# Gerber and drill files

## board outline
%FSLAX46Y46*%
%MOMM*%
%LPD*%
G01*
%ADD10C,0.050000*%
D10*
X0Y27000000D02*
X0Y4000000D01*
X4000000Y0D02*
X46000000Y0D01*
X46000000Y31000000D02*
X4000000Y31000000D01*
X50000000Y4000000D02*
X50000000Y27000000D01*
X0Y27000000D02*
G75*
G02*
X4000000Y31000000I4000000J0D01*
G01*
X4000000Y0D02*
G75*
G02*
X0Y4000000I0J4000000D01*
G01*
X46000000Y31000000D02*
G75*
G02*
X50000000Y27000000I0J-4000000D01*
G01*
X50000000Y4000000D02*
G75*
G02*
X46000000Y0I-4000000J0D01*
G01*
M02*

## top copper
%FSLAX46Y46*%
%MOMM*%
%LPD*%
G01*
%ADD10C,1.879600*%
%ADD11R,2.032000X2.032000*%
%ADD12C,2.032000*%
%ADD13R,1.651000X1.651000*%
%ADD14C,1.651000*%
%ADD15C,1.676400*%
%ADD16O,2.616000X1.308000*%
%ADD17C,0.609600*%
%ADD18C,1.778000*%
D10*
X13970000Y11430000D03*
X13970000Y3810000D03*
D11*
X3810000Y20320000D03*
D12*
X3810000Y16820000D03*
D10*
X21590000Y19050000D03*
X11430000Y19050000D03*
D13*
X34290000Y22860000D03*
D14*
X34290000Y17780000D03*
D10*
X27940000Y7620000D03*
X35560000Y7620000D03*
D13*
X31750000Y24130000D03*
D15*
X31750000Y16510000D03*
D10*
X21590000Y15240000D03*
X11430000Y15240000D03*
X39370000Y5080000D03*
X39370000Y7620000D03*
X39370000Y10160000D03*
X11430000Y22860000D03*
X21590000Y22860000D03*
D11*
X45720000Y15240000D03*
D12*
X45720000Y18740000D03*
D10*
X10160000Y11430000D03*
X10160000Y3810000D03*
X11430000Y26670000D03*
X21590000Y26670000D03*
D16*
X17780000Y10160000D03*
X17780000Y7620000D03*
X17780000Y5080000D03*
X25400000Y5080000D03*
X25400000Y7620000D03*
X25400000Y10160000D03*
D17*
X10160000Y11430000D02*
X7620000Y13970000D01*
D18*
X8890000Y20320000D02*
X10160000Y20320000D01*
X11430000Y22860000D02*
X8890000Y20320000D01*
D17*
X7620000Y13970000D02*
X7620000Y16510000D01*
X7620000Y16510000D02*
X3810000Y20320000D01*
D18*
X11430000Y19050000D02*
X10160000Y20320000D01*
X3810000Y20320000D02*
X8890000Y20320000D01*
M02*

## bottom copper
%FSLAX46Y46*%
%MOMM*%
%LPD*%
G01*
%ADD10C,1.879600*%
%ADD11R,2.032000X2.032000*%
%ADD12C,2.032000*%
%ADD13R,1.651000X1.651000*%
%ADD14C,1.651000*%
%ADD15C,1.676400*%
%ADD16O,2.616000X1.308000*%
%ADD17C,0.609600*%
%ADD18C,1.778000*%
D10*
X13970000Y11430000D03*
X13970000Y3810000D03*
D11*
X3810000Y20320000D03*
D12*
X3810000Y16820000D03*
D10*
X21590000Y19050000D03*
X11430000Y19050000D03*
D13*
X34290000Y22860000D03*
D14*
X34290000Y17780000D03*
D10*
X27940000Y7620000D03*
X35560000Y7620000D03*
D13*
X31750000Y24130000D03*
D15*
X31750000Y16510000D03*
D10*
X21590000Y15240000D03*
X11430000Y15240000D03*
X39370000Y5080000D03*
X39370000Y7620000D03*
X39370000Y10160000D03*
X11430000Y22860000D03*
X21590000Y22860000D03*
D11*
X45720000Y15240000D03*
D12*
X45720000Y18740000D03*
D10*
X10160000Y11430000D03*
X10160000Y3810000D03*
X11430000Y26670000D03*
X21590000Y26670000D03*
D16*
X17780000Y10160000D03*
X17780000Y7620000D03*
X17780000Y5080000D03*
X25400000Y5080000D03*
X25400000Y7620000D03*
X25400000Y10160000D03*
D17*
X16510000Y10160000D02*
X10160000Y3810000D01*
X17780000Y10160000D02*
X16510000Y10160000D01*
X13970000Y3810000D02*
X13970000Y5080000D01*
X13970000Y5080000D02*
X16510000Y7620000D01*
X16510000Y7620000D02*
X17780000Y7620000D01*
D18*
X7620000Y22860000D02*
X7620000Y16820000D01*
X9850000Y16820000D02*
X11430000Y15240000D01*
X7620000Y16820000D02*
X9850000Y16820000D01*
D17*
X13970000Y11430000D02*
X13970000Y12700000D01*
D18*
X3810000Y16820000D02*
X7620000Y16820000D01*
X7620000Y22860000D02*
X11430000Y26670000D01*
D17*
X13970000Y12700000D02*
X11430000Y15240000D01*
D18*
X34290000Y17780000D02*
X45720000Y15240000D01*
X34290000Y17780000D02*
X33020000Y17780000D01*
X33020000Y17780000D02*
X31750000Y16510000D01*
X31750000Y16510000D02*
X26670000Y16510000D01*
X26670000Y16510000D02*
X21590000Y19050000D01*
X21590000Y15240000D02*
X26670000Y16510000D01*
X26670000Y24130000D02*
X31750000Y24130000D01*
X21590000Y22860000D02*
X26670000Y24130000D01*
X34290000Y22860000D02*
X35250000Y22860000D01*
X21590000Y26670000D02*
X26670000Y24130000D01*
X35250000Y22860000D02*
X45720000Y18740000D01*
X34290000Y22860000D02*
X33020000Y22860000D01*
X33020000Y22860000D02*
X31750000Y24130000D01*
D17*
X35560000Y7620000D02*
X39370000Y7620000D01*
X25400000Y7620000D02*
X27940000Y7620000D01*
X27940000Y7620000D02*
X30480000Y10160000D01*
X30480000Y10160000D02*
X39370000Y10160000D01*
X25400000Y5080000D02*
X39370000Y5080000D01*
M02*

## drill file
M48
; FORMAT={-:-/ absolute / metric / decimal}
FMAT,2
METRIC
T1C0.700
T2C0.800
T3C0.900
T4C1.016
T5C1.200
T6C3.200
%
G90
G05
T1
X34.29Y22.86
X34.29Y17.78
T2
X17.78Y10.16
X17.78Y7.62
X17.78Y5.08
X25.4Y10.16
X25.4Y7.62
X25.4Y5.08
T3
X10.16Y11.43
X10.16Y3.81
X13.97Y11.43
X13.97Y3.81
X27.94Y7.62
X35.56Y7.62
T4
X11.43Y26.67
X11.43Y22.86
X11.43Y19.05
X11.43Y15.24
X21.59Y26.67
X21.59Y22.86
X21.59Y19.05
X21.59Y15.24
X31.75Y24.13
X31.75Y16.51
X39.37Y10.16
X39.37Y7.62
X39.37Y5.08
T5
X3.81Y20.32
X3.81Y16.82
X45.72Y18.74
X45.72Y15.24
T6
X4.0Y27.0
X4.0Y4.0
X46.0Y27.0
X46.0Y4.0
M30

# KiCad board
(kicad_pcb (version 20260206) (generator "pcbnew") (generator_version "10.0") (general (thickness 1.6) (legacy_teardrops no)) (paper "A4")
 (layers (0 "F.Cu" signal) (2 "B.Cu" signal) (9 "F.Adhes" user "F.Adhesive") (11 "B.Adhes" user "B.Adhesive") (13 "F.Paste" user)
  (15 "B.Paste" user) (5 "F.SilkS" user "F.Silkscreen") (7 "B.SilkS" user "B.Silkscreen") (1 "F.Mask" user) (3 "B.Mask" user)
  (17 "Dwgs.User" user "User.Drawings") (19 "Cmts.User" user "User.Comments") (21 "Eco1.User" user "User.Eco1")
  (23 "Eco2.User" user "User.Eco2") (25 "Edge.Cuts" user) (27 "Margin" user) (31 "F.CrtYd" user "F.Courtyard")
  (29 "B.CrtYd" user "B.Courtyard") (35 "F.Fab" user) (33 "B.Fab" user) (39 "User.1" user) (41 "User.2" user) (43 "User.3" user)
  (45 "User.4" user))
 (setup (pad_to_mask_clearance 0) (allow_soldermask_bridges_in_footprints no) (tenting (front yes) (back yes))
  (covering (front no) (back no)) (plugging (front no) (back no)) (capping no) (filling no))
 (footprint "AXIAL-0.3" (layer "F.Cu") (at 13.97 -7.62 -90)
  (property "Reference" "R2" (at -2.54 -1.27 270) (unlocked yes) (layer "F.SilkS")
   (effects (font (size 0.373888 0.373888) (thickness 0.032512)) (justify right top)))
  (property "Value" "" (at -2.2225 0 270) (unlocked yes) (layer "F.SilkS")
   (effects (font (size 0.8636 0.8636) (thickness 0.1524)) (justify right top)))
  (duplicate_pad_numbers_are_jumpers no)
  (pad "P$1" thru_hole circle (at -3.81 0 270) (size 1.8796 1.8796) (drill 0.9) (layers "*.Cu" "*.Mask") (remove_unused_layers no)
   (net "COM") (solder_mask_margin 0.1016) (thermal_bridge_angle 0))
  (pad "P$2" thru_hole circle (at 3.81 0 270) (size 1.8796 1.8796) (drill 0.9) (layers "*.Cu" "*.Mask") (remove_unused_layers no) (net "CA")
   (solder_mask_margin 0.1016) (thermal_bridge_angle 0)))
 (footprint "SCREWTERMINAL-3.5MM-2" (layer "F.Cu") (at 3.81 -20.32 -90)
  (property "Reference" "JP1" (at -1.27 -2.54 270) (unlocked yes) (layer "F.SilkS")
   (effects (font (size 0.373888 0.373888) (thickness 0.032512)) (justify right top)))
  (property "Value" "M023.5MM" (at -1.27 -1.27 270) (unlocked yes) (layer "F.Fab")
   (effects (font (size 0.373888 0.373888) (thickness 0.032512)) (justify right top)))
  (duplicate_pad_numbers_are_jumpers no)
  (pad "1" thru_hole rect (at 0 0 270) (size 2.032 2.032) (drill 1.2) (layers "*.Cu" "*.Mask") (remove_unused_layers no) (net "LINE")
   (solder_mask_margin 0.1016) (thermal_bridge_angle 0))
  (pad "2" thru_hole circle (at 3.5 0 270) (size 2.032 2.032) (drill 1.2) (layers "*.Cu" "*.Mask") (remove_unused_layers no) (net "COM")
   (solder_mask_margin 0.1016) (thermal_bridge_angle 0)))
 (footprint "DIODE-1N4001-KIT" (layer "F.Cu") (at 16.51 -19.05 180)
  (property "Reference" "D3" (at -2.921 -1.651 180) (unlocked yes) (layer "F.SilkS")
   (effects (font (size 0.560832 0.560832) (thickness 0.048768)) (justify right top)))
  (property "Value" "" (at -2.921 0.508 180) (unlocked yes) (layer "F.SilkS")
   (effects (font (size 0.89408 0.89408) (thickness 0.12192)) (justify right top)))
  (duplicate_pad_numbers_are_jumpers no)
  (pad "A" thru_hole circle (at -5.08 0 180) (size 1.8796 1.8796) (drill 1.016) (layers "*.Cu") (remove_unused_layers no) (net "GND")
   (solder_mask_margin 0.1016) (thermal_bridge_angle 0))
  (pad "C" thru_hole circle (at 5.08 0 180) (size 1.8796 1.8796) (drill 1.016) (layers "*.Cu") (remove_unused_layers no) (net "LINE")
   (solder_mask_margin 0.1016) (thermal_bridge_angle 0)))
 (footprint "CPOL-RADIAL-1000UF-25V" (layer "F.Cu") (at 34.29 -20.32 90)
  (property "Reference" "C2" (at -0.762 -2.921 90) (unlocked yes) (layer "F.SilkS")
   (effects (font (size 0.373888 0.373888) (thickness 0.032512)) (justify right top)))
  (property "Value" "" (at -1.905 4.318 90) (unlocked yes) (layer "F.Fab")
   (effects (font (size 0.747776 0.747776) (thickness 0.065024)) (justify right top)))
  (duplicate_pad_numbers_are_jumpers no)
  (pad "1" thru_hole rect (at 2.54 0 90) (size 1.651 1.651) (drill 0.7) (layers "*.Cu" "*.Mask") (remove_unused_layers no) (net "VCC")
   (solder_mask_margin 0.1016) (thermal_bridge_angle 0))
  (pad "2" thru_hole circle (at -2.54 0 90) (size 1.651 1.651) (drill 0.7) (layers "*.Cu" "*.Mask") (remove_unused_layers no) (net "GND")
   (solder_mask_margin 0.1016) (thermal_bridge_angle 0)))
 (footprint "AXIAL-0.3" (layer "F.Cu") (at 31.75 -7.62)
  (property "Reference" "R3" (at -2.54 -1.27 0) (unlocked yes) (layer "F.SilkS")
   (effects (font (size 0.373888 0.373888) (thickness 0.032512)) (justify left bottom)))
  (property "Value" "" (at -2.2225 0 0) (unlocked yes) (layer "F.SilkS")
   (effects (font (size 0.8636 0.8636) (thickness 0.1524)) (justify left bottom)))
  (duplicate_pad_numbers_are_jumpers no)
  (pad "P$1" thru_hole circle (at -3.81 0) (size 1.8796 1.8796) (drill 0.9) (layers "*.Cu" "*.Mask") (remove_unused_layers no) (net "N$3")
   (solder_mask_margin 0.1016) (thermal_bridge_angle 0))
  (pad "P$2" thru_hole circle (at 3.81 0) (size 1.8796 1.8796) (drill 0.9) (layers "*.Cu" "*.Mask") (remove_unused_layers no) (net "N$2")
   (solder_mask_margin 0.1016) (thermal_bridge_angle 0)))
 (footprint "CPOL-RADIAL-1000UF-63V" (layer "F.Cu") (at 31.75 -20.32 90)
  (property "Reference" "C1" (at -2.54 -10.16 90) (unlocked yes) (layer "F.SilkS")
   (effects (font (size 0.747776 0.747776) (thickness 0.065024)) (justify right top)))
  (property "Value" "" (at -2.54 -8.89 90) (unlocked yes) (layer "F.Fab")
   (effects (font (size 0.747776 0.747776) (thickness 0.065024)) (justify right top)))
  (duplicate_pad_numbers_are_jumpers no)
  (pad "1" thru_hole rect (at 3.81 0 90) (size 1.651 1.651) (drill 1.016) (layers "*.Cu" "*.Mask") (remove_unused_layers no) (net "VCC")
   (solder_mask_margin 0.1016) (thermal_bridge_angle 0))
  (pad "2" thru_hole circle (at -3.81 0 90) (size 1.6764 1.6764) (drill 1.016) (layers "*.Cu" "*.Mask") (remove_unused_layers no)
   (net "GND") (solder_mask_margin 0.1016) (thermal_bridge_angle 0)))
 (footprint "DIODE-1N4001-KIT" (layer "F.Cu") (at 16.51 -15.24 180)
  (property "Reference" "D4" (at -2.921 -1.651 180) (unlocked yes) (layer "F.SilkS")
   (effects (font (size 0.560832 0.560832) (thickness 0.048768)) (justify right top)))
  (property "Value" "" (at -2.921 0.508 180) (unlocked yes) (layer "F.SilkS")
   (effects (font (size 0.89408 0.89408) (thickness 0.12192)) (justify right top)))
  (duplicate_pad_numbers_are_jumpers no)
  (pad "A" thru_hole circle (at -5.08 0 180) (size 1.8796 1.8796) (drill 1.016) (layers "*.Cu") (remove_unused_layers no) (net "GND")
   (solder_mask_margin 0.1016) (thermal_bridge_angle 0))
  (pad "C" thru_hole circle (at 5.08 0 180) (size 1.8796 1.8796) (drill 1.016) (layers "*.Cu") (remove_unused_layers no) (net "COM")
   (solder_mask_margin 0.1016) (thermal_bridge_angle 0)))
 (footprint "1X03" (layer "F.Cu") (at 39.37 -5.08 90)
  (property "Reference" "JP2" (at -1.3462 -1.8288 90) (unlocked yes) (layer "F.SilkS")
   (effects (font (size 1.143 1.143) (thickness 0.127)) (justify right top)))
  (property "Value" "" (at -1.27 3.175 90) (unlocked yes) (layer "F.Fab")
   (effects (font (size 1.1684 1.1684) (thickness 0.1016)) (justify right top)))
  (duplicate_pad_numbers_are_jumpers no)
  (pad "1" thru_hole circle (at 0 0 180) (size 1.8796 1.8796) (drill 1.016) (layers "*.Cu" "*.Mask") (remove_unused_layers no) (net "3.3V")
   (solder_mask_margin 0.1016) (thermal_bridge_angle 0))
  (pad "2" thru_hole circle (at 2.54 0 180) (size 1.8796 1.8796) (drill 1.016) (layers "*.Cu" "*.Mask") (remove_unused_layers no)
   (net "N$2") (solder_mask_margin 0.1016) (thermal_bridge_angle 0))
  (pad "3" thru_hole circle (at 5.08 0 180) (size 1.8796 1.8796) (drill 1.016) (layers "*.Cu" "*.Mask") (remove_unused_layers no)
   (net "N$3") (solder_mask_margin 0.1016) (thermal_bridge_angle 0)))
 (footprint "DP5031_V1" (layer "F.Cu") (at 0 0)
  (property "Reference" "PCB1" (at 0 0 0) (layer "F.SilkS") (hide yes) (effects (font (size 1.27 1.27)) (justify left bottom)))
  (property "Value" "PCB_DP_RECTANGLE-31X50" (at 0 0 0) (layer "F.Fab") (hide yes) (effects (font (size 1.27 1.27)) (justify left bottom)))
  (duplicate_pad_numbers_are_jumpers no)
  (fp_line (start 0 -27) (end 0 -4) (stroke (width 0.05) (type solid)) (layer "Edge.Cuts"))
  (fp_line (start 4 0) (end 46 0) (stroke (width 0.05) (type solid)) (layer "Edge.Cuts"))
  (fp_line (start 46 -31) (end 4 -31) (stroke (width 0.05) (type solid)) (layer "Edge.Cuts"))
  (fp_line (start 50 -4) (end 50 -27) (stroke (width 0.05) (type solid)) (layer "Edge.Cuts"))
  (fp_arc (start 0 -27) (mid 1.171573 -29.828427) (end 4 -31) (stroke (width 0.05) (type solid)) (layer "Edge.Cuts"))
  (fp_arc (start 4 0) (mid 1.171573 -1.171573) (end 0 -4) (stroke (width 0.05) (type solid)) (layer "Edge.Cuts"))
  (fp_arc (start 46 -31) (mid 48.828427 -29.828427) (end 50 -27) (stroke (width 0.05) (type solid)) (layer "Edge.Cuts"))
  (fp_arc (start 50 -4) (mid 48.828427 -1.171573) (end 46 0) (stroke (width 0.05) (type solid)) (layer "Edge.Cuts"))
  (pad "" np_thru_hole circle (at 4 -27) (size 3.2 3.2) (drill 3.2) (layers "*.Cu" "*.Mask"))
  (pad "" np_thru_hole circle (at 4 -4) (size 3.2 3.2) (drill 3.2) (layers "*.Cu" "*.Mask"))
  (pad "" np_thru_hole circle (at 46 -27) (size 3.2 3.2) (drill 3.2) (layers "*.Cu" "*.Mask"))
  (pad "" np_thru_hole circle (at 46 -4) (size 3.2 3.2) (drill 3.2) (layers "*.Cu" "*.Mask"))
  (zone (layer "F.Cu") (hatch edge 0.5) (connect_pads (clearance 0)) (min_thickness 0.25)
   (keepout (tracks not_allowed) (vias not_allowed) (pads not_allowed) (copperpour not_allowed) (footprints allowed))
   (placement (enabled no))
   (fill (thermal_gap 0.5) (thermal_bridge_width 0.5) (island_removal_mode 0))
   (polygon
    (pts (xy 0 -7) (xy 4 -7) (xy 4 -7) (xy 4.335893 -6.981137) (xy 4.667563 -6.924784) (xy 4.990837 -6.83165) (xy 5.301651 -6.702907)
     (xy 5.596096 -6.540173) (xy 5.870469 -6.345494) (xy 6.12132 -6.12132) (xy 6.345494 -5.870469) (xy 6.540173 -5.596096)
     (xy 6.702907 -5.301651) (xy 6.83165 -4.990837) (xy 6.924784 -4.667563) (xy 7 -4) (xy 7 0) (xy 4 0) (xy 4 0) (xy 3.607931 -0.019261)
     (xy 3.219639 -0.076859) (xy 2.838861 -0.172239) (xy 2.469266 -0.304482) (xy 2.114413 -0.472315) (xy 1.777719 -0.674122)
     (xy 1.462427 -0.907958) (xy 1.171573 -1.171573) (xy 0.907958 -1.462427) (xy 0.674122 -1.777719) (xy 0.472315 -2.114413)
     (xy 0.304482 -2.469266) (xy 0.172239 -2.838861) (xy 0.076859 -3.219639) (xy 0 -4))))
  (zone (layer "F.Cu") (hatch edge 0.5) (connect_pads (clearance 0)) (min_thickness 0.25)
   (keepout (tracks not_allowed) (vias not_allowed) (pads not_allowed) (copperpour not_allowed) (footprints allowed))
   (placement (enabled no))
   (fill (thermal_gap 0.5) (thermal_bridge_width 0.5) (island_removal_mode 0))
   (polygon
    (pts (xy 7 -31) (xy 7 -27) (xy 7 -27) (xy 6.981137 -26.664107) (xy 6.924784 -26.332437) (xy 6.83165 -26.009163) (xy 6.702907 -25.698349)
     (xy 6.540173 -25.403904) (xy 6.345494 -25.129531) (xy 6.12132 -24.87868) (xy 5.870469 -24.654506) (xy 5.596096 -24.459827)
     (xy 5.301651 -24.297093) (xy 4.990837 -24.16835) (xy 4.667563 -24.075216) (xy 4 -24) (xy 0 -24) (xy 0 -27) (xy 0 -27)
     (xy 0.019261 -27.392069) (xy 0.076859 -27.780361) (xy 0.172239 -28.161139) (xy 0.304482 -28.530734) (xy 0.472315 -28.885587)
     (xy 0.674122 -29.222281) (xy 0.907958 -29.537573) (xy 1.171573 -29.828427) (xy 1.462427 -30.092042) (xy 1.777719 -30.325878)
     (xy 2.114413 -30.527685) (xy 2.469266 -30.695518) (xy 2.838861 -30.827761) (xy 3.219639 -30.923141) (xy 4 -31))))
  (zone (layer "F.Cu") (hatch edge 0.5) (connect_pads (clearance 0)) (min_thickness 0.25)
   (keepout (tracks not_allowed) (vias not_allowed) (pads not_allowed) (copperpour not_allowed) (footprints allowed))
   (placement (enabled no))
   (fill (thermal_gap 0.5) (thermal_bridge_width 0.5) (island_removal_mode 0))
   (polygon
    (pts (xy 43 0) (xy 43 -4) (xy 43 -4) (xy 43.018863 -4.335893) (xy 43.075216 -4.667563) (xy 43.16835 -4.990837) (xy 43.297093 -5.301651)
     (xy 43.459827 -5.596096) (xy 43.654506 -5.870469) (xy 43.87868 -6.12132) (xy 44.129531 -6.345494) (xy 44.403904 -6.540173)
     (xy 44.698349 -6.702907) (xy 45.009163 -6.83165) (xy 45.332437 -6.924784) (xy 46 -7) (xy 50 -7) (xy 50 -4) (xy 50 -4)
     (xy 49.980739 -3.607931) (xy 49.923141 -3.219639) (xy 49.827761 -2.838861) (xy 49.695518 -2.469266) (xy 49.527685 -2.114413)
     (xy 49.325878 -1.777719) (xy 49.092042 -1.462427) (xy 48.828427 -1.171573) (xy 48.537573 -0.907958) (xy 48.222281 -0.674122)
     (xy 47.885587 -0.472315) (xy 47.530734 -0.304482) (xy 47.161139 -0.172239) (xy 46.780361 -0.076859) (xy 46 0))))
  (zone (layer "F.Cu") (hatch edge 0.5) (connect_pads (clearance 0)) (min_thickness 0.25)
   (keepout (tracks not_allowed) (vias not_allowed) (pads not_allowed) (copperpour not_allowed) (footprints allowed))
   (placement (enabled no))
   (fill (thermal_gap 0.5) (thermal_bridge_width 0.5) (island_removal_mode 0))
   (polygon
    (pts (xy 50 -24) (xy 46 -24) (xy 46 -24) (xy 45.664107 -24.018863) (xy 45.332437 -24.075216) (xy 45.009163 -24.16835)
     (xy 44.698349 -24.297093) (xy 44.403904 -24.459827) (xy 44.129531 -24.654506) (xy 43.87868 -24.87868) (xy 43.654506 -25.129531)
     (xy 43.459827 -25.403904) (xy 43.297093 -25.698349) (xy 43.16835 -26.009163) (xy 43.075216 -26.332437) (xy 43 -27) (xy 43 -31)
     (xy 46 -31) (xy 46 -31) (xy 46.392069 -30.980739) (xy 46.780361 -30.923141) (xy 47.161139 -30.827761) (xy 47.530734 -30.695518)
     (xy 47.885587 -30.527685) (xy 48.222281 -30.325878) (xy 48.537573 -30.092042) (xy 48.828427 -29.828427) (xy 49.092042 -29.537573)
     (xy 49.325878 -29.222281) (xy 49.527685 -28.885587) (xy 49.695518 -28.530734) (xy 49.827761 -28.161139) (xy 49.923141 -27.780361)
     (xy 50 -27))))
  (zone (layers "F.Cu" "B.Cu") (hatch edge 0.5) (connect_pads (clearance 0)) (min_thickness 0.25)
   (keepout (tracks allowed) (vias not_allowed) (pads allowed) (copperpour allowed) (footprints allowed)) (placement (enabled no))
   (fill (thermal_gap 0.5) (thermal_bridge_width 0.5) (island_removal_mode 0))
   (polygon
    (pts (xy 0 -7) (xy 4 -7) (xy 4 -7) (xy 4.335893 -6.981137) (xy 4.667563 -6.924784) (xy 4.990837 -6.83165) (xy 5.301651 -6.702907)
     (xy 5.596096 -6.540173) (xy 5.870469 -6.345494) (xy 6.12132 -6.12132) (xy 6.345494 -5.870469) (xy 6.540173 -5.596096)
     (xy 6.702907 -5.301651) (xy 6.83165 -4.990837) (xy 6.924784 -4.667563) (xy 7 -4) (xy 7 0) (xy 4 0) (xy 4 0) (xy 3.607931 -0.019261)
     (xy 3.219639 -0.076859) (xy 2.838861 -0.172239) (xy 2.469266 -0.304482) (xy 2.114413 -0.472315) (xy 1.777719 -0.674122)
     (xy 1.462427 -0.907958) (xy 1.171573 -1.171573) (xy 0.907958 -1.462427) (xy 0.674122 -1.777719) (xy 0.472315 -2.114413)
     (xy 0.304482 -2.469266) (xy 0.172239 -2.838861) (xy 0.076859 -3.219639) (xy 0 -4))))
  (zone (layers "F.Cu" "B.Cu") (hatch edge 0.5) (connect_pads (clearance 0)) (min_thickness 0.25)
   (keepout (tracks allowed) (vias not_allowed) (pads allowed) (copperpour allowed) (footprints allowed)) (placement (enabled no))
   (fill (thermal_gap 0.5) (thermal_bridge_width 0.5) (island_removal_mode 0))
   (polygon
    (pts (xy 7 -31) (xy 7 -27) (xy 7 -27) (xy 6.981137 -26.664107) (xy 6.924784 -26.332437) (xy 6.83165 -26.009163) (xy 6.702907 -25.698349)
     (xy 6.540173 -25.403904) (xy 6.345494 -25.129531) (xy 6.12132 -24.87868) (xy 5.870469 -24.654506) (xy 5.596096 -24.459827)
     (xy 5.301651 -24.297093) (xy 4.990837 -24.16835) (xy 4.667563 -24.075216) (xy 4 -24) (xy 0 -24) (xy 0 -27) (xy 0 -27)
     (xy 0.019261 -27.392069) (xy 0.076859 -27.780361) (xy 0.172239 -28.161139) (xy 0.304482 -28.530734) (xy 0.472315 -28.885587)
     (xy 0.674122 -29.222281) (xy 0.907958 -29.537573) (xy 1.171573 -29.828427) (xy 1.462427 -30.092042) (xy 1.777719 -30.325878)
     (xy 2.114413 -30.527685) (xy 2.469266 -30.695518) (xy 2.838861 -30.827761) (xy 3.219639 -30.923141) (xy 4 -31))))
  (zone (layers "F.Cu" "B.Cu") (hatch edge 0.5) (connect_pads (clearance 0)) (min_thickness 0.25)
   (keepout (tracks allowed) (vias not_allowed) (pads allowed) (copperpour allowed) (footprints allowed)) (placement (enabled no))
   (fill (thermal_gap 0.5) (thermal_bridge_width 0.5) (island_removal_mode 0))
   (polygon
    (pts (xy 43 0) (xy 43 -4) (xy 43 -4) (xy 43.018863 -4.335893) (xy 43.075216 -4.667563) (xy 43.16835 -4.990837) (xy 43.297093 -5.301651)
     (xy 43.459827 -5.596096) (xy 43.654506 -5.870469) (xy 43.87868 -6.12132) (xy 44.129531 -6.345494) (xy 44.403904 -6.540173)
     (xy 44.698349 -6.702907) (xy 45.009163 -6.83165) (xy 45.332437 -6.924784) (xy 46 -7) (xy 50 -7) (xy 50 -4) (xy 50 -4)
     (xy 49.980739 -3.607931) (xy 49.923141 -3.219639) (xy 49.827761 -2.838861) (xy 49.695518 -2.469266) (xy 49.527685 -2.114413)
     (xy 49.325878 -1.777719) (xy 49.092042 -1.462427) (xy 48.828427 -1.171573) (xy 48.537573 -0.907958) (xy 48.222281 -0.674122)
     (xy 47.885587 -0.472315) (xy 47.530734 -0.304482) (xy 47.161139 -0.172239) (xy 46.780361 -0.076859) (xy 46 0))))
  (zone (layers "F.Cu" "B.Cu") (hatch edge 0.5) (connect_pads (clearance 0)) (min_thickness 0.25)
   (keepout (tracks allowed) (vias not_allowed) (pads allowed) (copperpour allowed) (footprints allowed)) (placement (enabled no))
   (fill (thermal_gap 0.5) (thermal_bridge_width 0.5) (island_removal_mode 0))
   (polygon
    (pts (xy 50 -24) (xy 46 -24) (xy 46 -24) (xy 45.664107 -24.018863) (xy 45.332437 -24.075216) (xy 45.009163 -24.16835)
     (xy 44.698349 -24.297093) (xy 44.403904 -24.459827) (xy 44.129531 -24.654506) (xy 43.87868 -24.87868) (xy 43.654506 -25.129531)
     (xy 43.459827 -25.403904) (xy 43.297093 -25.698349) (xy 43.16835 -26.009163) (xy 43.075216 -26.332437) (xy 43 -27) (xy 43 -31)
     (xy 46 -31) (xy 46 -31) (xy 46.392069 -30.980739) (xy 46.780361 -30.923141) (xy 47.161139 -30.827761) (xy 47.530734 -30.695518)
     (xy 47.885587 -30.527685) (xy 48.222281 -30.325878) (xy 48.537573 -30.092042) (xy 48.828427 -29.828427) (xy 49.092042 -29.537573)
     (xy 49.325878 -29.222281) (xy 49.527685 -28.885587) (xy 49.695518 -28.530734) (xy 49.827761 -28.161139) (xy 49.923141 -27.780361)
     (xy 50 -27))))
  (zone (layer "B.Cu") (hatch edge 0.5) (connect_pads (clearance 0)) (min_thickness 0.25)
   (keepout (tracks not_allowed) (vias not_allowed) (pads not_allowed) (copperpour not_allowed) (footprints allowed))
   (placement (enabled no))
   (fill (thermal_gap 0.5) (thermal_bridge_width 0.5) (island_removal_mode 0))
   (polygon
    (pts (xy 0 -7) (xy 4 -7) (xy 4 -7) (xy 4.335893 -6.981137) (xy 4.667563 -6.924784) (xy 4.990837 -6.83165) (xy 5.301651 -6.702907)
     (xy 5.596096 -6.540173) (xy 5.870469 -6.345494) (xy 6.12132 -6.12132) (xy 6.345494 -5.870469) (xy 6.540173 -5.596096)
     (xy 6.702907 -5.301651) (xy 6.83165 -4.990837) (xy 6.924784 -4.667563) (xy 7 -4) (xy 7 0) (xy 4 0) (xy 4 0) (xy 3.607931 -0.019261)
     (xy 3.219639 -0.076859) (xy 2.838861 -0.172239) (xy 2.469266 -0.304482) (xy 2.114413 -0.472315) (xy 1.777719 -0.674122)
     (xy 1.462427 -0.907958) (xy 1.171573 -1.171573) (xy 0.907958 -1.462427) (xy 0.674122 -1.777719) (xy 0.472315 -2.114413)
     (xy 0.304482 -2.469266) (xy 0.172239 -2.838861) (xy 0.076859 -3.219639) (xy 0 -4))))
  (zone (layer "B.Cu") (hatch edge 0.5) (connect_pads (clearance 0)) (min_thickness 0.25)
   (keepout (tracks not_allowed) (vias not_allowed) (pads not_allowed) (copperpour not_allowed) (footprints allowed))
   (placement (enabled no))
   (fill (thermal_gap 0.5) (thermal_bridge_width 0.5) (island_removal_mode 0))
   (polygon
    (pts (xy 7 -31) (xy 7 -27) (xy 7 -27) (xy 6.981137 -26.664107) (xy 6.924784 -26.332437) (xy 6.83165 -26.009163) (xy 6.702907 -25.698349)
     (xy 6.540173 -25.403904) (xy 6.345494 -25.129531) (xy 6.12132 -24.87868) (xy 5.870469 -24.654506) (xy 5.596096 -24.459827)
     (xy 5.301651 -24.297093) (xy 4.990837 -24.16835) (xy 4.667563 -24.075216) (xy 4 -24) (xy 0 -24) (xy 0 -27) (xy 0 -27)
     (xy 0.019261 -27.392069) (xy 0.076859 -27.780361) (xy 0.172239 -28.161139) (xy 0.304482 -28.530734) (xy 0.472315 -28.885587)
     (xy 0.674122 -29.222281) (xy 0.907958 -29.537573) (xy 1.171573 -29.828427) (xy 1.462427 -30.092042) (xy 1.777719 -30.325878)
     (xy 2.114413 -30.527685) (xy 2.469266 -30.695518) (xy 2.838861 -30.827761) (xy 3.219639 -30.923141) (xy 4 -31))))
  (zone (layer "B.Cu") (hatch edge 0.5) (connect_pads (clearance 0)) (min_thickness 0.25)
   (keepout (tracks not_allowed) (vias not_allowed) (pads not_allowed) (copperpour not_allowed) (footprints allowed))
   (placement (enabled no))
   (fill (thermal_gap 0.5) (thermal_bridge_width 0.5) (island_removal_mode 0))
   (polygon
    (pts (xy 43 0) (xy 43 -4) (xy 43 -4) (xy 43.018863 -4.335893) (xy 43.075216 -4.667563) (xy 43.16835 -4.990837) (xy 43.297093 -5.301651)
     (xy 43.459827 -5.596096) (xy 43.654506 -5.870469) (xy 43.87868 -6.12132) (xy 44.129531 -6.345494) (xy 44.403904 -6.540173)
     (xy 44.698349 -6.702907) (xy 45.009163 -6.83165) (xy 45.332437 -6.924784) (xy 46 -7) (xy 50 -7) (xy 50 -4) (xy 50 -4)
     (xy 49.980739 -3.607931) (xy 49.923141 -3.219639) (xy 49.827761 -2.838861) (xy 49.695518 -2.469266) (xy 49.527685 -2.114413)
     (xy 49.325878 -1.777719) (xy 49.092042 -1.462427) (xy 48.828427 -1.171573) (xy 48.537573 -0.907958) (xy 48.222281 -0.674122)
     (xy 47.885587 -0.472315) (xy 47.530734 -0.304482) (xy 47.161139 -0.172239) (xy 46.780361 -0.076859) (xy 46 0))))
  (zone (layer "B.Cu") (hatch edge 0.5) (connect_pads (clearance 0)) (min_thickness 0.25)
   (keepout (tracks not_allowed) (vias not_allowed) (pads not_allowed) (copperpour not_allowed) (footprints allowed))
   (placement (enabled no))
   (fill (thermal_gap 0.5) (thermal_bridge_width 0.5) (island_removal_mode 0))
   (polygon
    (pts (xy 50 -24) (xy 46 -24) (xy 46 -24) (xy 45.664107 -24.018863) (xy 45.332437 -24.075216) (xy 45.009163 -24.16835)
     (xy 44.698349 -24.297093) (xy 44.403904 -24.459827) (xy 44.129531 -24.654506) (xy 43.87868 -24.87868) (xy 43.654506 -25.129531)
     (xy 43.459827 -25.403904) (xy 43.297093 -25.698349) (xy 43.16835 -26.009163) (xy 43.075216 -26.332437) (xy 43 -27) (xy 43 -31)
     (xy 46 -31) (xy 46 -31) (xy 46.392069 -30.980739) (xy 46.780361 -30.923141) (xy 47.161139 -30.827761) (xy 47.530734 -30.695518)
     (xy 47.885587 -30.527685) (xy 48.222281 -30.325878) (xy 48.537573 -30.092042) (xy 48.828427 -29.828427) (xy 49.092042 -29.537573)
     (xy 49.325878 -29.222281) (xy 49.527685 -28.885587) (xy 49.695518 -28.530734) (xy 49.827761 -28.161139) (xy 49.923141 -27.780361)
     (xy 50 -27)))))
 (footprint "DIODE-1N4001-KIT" (layer "F.Cu") (at 16.51 -22.86)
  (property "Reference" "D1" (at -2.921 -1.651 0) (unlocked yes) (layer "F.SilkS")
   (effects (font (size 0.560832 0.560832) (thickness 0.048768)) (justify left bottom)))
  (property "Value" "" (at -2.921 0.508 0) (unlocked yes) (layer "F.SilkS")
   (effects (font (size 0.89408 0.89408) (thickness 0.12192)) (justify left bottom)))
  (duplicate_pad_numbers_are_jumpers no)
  (pad "A" thru_hole circle (at -5.08 0) (size 1.8796 1.8796) (drill 1.016) (layers "*.Cu") (remove_unused_layers no) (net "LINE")
   (solder_mask_margin 0.1016) (thermal_bridge_angle 0))
  (pad "C" thru_hole circle (at 5.08 0) (size 1.8796 1.8796) (drill 1.016) (layers "*.Cu") (remove_unused_layers no) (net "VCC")
   (solder_mask_margin 0.1016) (thermal_bridge_angle 0)))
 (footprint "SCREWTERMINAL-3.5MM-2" (layer "F.Cu") (at 45.72 -15.24 90)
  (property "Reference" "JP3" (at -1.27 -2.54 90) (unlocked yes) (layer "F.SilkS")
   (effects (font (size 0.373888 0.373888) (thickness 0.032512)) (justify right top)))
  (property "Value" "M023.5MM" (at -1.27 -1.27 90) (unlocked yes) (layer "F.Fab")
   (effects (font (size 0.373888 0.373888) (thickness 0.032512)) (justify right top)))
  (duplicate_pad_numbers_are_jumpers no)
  (pad "1" thru_hole rect (at 0 0 90) (size 2.032 2.032) (drill 1.2) (layers "*.Cu" "*.Mask") (remove_unused_layers no) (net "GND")
   (solder_mask_margin 0.1016) (thermal_bridge_angle 0))
  (pad "2" thru_hole circle (at 3.5 0 90) (size 2.032 2.032) (drill 1.2) (layers "*.Cu" "*.Mask") (remove_unused_layers no) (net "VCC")
   (solder_mask_margin 0.1016) (thermal_bridge_angle 0)))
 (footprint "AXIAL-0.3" (layer "F.Cu") (at 10.16 -7.62 -90)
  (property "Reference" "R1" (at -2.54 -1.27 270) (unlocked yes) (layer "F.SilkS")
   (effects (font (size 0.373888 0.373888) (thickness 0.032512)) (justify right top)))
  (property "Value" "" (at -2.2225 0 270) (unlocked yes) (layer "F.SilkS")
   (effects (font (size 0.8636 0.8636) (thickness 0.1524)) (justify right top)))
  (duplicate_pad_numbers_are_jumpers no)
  (pad "P$1" thru_hole circle (at -3.81 0 270) (size 1.8796 1.8796) (drill 0.9) (layers "*.Cu" "*.Mask") (remove_unused_layers no)
   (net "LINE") (solder_mask_margin 0.1016) (thermal_bridge_angle 0))
  (pad "P$2" thru_hole circle (at 3.81 0 270) (size 1.8796 1.8796) (drill 0.9) (layers "*.Cu" "*.Mask") (remove_unused_layers no) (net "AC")
   (solder_mask_margin 0.1016) (thermal_bridge_angle 0)))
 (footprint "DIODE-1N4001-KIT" (layer "F.Cu") (at 16.51 -26.67)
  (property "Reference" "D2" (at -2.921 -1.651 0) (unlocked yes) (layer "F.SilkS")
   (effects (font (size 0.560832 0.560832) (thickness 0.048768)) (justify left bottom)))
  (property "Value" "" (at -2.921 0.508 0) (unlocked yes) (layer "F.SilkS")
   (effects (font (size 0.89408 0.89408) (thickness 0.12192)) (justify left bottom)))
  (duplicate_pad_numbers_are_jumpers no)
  (pad "A" thru_hole circle (at -5.08 0) (size 1.8796 1.8796) (drill 1.016) (layers "*.Cu") (remove_unused_layers no) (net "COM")
   (solder_mask_margin 0.1016) (thermal_bridge_angle 0))
  (pad "C" thru_hole circle (at 5.08 0) (size 1.8796 1.8796) (drill 1.016) (layers "*.Cu") (remove_unused_layers no) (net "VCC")
   (solder_mask_margin 0.1016) (thermal_bridge_angle 0)))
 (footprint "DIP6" (layer "F.Cu") (at 21.59 -7.62)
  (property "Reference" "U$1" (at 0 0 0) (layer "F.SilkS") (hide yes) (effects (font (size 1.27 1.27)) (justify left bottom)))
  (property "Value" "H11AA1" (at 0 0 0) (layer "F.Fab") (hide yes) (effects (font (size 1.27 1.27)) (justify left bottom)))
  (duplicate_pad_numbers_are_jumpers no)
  (pad "1" thru_hole oval (at -3.81 -2.54) (size 2.616 1.308) (drill 0.8) (layers "*.Cu" "*.Mask") (remove_unused_layers no) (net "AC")
   (solder_mask_margin 0.1016) (thermal_bridge_angle 0))
  (pad "2" thru_hole oval (at -3.81 0) (size 2.616 1.308) (drill 0.8) (layers "*.Cu" "*.Mask") (remove_unused_layers no) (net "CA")
   (solder_mask_margin 0.1016) (thermal_bridge_angle 0))
  (pad "3" thru_hole oval (at -3.81 2.54) (size 2.616 1.308) (drill 0.8) (layers "*.Cu" "*.Mask") (remove_unused_layers no)
   (solder_mask_margin 0.1016) (thermal_bridge_angle 0))
  (pad "4" thru_hole oval (at 3.81 2.54) (size 2.616 1.308) (drill 0.8) (layers "*.Cu" "*.Mask") (remove_unused_layers no) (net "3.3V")
   (solder_mask_margin 0.1016) (thermal_bridge_angle 0))
  (pad "5" thru_hole oval (at 3.81 0) (size 2.616 1.308) (drill 0.8) (layers "*.Cu" "*.Mask") (remove_unused_layers no) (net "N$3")
   (solder_mask_margin 0.1016) (thermal_bridge_angle 0))
  (pad "6" thru_hole oval (at 3.81 -2.54) (size 2.616 1.308) (drill 0.8) (layers "*.Cu" "*.Mask") (remove_unused_layers no)
   (solder_mask_margin 0.1016) (thermal_bridge_angle 0)))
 (segment (start 16.51 -10.16) (end 10.16 -3.81) (width 0.6096) (layer "B.Cu") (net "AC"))
 (segment (start 17.78 -10.16) (end 16.51 -10.16) (width 0.6096) (layer "B.Cu") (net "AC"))
 (segment (start 13.97 -3.81) (end 13.97 -5.08) (width 0.6096) (layer "B.Cu") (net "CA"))
 (segment (start 13.97 -5.08) (end 16.51 -7.62) (width 0.6096) (layer "B.Cu") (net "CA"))
 (segment (start 16.51 -7.62) (end 17.78 -7.62) (width 0.6096) (layer "B.Cu") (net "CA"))
 (segment (start 10.16 -11.43) (end 7.62 -13.97) (width 0.6096) (layer "F.Cu") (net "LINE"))
 (segment (start 8.89 -20.32) (end 10.16 -20.32) (width 1.778) (layer "F.Cu") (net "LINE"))
 (segment (start 11.43 -22.86) (end 8.89 -20.32) (width 1.778) (layer "F.Cu") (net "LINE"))
 (segment (start 7.62 -13.97) (end 7.62 -16.51) (width 0.6096) (layer "F.Cu") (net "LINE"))
 (segment (start 7.62 -16.51) (end 3.81 -20.32) (width 0.6096) (layer "F.Cu") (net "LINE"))
 (segment (start 11.43 -19.05) (end 10.16 -20.32) (width 1.778) (layer "F.Cu") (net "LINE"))
 (segment (start 3.81 -20.32) (end 8.89 -20.32) (width 1.778) (layer "F.Cu") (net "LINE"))
 (segment (start 7.62 -22.86) (end 7.62 -16.82) (width 1.778) (layer "B.Cu") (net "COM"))
 (segment (start 9.85 -16.82) (end 11.43 -15.24) (width 1.778) (layer "B.Cu") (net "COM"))
 (segment (start 7.62 -16.82) (end 9.85 -16.82) (width 1.778) (layer "B.Cu") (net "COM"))
 (segment (start 13.97 -11.43) (end 13.97 -12.7) (width 0.6096) (layer "B.Cu") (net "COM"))
 (segment (start 3.81 -16.82) (end 7.62 -16.82) (width 1.778) (layer "B.Cu") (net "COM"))
 (segment (start 7.62 -22.86) (end 11.43 -26.67) (width 1.778) (layer "B.Cu") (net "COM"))
 (segment (start 13.97 -12.7) (end 11.43 -15.24) (width 0.6096) (layer "B.Cu") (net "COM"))
 (segment (start 34.29 -17.78) (end 45.72 -15.24) (width 1.778) (layer "B.Cu") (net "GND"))
 (segment (start 34.29 -17.78) (end 33.02 -17.78) (width 1.778) (layer "B.Cu") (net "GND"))
 (segment (start 33.02 -17.78) (end 31.75 -16.51) (width 1.778) (layer "B.Cu") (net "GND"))
 (segment (start 31.75 -16.51) (end 26.67 -16.51) (width 1.778) (layer "B.Cu") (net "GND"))
 (segment (start 26.67 -16.51) (end 21.59 -19.05) (width 1.778) (layer "B.Cu") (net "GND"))
 (segment (start 21.59 -15.24) (end 26.67 -16.51) (width 1.778) (layer "B.Cu") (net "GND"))
 (segment (start 26.67 -24.13) (end 31.75 -24.13) (width 1.778) (layer "B.Cu") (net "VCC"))
 (segment (start 21.59 -22.86) (end 26.67 -24.13) (width 1.778) (layer "B.Cu") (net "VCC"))
 (segment (start 34.29 -22.86) (end 35.25 -22.86) (width 1.778) (layer "B.Cu") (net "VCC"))
 (segment (start 21.59 -26.67) (end 26.67 -24.13) (width 1.778) (layer "B.Cu") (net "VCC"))
 (segment (start 35.25 -22.86) (end 45.72 -18.74) (width 1.778) (layer "B.Cu") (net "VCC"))
 (segment (start 34.29 -22.86) (end 33.02 -22.86) (width 1.778) (layer "B.Cu") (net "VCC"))
 (segment (start 33.02 -22.86) (end 31.75 -24.13) (width 1.778) (layer "B.Cu") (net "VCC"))
 (segment (start 35.56 -7.62) (end 39.37 -7.62) (width 0.6096) (layer "B.Cu") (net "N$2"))
 (segment (start 25.4 -7.62) (end 27.94 -7.62) (width 0.6096) (layer "B.Cu") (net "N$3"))
 (segment (start 27.94 -7.62) (end 30.48 -10.16) (width 0.6096) (layer "B.Cu") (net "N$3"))
 (segment (start 30.48 -10.16) (end 39.37 -10.16) (width 0.6096) (layer "B.Cu") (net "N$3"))
 (segment (start 25.4 -5.08) (end 39.37 -5.08) (width 0.6096) (layer "B.Cu") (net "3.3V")))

